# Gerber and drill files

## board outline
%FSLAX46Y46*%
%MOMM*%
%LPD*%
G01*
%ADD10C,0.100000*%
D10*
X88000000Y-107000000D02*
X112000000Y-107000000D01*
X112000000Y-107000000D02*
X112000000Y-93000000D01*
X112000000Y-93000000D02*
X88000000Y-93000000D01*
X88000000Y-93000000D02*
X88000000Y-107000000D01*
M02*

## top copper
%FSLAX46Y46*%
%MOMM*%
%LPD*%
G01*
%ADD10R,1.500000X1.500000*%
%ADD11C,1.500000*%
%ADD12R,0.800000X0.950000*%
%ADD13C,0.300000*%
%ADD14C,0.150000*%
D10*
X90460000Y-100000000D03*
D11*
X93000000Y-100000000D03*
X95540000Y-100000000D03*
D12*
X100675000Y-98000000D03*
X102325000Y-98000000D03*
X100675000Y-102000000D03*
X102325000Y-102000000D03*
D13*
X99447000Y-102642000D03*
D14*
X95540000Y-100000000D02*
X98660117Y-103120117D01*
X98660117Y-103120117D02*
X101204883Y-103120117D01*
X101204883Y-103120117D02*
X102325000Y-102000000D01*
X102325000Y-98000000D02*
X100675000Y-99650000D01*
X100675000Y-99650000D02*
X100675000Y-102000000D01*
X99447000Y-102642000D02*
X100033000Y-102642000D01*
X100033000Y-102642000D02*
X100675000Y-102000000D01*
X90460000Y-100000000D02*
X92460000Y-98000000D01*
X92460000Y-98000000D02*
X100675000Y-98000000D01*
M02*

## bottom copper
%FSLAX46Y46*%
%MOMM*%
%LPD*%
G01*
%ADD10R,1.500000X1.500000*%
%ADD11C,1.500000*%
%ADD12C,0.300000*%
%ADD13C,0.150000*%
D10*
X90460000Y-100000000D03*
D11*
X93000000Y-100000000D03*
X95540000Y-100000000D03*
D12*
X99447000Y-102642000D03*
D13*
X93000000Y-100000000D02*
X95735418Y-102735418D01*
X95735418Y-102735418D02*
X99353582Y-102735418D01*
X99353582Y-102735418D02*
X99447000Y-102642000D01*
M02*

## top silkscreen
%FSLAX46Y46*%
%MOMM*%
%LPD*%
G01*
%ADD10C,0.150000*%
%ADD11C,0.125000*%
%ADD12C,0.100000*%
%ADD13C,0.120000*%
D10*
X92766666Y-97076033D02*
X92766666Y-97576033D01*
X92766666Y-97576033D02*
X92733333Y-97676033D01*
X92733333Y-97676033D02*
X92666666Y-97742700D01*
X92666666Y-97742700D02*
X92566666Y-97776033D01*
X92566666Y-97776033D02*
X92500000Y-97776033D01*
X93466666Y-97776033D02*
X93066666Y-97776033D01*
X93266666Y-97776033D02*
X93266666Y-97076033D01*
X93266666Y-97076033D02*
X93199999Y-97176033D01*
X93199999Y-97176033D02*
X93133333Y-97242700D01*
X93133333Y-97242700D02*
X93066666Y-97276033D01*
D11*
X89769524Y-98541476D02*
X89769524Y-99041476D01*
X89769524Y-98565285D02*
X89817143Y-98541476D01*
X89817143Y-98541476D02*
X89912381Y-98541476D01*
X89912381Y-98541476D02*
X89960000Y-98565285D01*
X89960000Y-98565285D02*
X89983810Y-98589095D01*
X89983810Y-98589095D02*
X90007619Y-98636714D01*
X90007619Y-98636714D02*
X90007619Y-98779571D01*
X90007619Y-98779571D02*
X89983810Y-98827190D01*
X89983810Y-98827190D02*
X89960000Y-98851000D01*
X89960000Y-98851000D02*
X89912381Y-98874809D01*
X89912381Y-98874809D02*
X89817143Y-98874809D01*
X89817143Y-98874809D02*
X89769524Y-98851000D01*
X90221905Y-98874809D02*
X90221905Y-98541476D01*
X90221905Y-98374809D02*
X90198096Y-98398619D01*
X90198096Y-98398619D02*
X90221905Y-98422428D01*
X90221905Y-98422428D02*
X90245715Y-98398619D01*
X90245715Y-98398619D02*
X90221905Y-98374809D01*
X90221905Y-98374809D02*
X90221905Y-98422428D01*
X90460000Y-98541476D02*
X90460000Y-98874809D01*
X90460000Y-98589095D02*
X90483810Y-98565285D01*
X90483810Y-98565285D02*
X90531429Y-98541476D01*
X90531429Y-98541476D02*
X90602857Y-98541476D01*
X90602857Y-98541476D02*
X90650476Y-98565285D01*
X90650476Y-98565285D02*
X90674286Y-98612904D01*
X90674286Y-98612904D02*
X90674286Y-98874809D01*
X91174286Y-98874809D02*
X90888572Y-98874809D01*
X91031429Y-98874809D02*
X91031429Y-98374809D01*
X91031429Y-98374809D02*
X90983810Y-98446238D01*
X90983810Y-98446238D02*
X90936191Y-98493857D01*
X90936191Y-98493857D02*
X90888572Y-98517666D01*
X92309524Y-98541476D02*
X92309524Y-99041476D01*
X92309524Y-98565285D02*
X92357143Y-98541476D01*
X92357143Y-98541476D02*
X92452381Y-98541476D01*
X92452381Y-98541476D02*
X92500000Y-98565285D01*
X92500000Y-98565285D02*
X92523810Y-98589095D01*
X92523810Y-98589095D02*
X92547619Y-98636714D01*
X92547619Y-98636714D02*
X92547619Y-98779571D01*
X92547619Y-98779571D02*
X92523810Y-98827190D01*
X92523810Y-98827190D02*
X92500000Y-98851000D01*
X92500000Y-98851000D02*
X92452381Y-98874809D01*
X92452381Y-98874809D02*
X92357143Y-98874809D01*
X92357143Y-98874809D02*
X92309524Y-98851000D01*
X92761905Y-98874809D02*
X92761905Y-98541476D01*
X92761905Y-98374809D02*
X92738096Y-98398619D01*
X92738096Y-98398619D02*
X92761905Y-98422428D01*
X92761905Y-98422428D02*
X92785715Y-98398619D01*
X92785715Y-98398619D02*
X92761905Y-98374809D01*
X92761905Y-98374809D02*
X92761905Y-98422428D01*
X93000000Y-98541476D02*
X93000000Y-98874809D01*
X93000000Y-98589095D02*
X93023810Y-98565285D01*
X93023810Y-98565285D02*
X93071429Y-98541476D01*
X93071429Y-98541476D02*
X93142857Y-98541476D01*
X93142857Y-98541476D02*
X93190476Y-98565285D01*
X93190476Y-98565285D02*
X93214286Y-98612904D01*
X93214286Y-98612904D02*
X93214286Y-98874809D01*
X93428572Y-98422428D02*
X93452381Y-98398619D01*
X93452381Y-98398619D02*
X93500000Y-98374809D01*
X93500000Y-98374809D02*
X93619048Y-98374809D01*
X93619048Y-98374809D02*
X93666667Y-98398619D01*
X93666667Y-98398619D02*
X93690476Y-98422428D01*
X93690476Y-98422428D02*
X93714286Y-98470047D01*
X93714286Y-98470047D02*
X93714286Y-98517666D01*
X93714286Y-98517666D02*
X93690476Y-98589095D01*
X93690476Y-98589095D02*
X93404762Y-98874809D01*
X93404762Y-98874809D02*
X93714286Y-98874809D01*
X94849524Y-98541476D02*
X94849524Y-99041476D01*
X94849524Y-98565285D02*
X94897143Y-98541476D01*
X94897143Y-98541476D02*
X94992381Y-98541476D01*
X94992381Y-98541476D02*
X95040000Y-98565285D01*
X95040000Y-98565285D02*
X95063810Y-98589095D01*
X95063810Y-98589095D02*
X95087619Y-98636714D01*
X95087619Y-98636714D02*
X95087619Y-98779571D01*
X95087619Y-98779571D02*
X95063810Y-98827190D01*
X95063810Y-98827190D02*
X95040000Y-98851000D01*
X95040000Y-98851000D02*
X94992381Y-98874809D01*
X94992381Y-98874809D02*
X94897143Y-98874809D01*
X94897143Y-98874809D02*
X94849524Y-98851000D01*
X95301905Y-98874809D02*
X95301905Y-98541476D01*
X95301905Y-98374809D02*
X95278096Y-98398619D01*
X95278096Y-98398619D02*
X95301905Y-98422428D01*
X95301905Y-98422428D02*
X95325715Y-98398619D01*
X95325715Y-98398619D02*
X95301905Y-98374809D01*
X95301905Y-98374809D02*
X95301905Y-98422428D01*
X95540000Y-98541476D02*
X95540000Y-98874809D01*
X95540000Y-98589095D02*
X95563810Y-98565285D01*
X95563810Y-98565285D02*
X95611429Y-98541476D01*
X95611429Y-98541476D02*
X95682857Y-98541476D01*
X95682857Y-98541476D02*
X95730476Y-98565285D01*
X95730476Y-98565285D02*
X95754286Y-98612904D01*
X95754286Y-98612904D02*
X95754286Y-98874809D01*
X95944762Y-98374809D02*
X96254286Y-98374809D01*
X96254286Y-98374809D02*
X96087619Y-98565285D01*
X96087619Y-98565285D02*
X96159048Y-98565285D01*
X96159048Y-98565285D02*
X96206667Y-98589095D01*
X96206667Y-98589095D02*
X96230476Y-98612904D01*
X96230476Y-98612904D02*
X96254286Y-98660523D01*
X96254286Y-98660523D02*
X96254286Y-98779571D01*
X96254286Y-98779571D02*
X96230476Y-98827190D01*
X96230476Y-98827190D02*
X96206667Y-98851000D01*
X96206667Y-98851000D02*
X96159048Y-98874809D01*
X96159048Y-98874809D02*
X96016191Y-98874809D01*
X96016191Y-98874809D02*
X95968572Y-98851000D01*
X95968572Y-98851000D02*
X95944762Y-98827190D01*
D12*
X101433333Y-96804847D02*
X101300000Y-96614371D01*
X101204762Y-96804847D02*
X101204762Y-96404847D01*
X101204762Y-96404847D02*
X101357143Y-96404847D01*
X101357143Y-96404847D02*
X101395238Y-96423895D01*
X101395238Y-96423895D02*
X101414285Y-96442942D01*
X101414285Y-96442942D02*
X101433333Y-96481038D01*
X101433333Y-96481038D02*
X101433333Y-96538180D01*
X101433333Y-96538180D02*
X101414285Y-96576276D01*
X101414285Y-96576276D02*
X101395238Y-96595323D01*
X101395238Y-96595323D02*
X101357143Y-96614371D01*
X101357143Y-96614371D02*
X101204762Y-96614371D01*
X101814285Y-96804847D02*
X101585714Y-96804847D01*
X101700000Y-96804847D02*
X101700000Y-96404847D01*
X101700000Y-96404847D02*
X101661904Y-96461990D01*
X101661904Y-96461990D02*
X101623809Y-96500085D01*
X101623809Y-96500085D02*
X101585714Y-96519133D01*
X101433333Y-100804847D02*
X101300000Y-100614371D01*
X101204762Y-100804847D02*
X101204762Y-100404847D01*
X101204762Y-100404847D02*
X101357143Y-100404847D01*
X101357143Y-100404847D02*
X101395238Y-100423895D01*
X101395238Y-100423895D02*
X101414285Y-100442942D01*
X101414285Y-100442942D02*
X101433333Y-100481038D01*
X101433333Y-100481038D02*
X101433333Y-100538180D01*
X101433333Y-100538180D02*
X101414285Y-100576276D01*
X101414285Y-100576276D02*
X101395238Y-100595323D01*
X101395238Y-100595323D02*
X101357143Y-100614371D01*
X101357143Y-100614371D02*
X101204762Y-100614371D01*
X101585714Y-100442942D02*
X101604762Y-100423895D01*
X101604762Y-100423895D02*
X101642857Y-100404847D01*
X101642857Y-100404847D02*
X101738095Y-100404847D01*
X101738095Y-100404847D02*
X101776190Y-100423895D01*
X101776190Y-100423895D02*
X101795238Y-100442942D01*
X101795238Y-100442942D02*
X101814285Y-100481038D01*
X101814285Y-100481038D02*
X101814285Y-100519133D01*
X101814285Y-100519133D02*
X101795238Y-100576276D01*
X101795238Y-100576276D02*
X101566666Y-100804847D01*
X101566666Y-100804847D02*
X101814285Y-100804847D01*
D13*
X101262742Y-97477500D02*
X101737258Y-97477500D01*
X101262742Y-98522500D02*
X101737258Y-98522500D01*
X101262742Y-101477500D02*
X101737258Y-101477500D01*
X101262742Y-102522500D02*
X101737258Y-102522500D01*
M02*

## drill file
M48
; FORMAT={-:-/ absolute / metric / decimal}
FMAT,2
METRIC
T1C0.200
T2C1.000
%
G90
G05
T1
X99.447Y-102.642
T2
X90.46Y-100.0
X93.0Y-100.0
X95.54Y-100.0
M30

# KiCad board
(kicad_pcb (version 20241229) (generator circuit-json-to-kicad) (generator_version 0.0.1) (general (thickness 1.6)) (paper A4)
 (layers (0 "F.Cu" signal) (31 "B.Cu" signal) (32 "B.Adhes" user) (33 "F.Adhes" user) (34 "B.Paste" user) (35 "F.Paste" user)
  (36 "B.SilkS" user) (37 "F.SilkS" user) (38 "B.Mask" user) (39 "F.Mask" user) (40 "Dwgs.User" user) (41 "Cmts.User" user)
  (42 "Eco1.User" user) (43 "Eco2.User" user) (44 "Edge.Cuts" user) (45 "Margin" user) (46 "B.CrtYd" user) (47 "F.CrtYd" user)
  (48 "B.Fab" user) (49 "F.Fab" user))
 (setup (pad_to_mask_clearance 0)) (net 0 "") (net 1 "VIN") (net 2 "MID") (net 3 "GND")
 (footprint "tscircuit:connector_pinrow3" (layer F.Cu) (at 93 100 0)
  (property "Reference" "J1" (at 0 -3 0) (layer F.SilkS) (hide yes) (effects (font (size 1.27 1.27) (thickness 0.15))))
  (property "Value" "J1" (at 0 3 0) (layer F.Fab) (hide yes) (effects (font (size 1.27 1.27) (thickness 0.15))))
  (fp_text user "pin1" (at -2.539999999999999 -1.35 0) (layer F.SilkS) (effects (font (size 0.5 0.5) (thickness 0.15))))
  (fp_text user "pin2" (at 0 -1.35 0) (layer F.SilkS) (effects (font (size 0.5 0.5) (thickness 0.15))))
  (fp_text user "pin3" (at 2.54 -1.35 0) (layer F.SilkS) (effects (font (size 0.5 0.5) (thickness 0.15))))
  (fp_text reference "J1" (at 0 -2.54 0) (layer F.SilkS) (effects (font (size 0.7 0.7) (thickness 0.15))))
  (pad "1" thru_hole rect (at -2.539999999999999 0 0) (size 1.5 1.5) (drill 1) (layers *.Cu *.Mask) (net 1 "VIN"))
  (pad "2" thru_hole circle (at 0 0 0) (size 1.5 1.5) (drill 1) (layers *.Cu *.Mask) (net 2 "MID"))
  (pad "3" thru_hole circle (at 2.54 0 0) (size 1.5 1.5) (drill 1) (layers *.Cu *.Mask) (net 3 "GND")))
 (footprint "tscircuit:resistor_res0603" (layer F.Cu) (at 101.5 98 0)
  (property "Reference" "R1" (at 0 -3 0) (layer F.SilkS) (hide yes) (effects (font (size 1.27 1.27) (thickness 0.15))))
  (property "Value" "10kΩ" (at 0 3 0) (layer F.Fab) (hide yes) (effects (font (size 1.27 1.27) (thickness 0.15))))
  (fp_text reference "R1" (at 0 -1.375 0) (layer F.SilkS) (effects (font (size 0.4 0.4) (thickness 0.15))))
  (fp_line (start -0.23725799999999997 -0.5225) (end 0.23725799999999997 -0.5225) (stroke (width 0.12) (type default)) (layer F.SilkS))
  (fp_line (start -0.23725799999999997 0.5225) (end 0.23725799999999997 0.5225) (stroke (width 0.12) (type default)) (layer F.SilkS))
  (pad "1" smd rect (at -0.825 0 0) (size 0.8 0.95) (layers F.Cu F.Mask) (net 1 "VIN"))
  (pad "2" smd rect (at 0.8250000000000002 0 0) (size 0.8 0.95) (layers F.Cu F.Mask) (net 2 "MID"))
  (pad "" smd rect (at -0.825 0 0) (size 0.5599999999999999 0.6649999999999999) (layers F.Paste))
  (pad "" smd rect (at 0.8250000000000002 0 0) (size 0.5599999999999999 0.6649999999999999) (layers F.Paste)))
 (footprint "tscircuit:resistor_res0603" (layer F.Cu) (at 101.5 102 0)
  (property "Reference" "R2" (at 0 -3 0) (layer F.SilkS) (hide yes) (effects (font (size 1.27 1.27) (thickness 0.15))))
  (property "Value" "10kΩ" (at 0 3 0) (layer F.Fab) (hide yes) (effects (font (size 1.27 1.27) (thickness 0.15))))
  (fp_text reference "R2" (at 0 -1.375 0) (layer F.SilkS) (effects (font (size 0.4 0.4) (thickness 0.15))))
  (fp_line (start -0.23725799999999997 -0.5225) (end 0.23725799999999997 -0.5225) (stroke (width 0.12) (type default)) (layer F.SilkS))
  (fp_line (start -0.23725799999999997 0.5225) (end 0.23725799999999997 0.5225) (stroke (width 0.12) (type default)) (layer F.SilkS))
  (pad "1" smd rect (at -0.825 0 0) (size 0.8 0.95) (layers F.Cu F.Mask) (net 2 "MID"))
  (pad "2" smd rect (at 0.8250000000000002 0 0) (size 0.8 0.95) (layers F.Cu F.Mask) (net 3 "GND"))
  (pad "" smd rect (at -0.825 0 0) (size 0.5599999999999999 0.6649999999999999) (layers F.Paste))
  (pad "" smd rect (at 0.8250000000000002 0 0) (size 0.5599999999999999 0.6649999999999999) (layers F.Paste)))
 (segment (start 95.54 100) (end 98.66011723078628 103.12011723078629) (width 0.15) (layer F.Cu) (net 3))
 (segment (start 98.66011723078628 103.12011723078629) (end 101.20488276921371 103.12011723078629) (width 0.15) (layer F.Cu) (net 3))
 (segment (start 101.20488276921371 103.12011723078629) (end 102.325 102) (width 0.15) (layer F.Cu) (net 3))
 (segment (start 102.325 98) (end 100.675 99.65) (width 0.15) (layer F.Cu) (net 2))
 (segment (start 100.675 99.65) (end 100.675 102) (width 0.15) (layer F.Cu) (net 2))
 (segment (start 93 100) (end 95.73541811585916 102.73541811585916) (width 0.15) (layer B.Cu) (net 2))
 (segment (start 95.73541811585916 102.73541811585916) (end 99.35358188414084 102.73541811585916) (width 0.15) (layer B.Cu) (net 2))
 (segment (start 99.35358188414084 102.73541811585916) (end 99.447 102.642) (width 0.15) (layer B.Cu) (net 2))
 (segment (start 99.447 102.642) (end 100.033 102.642) (width 0.15) (layer F.Cu) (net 2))
 (segment (start 100.033 102.642) (end 100.675 102) (width 0.15) (layer F.Cu) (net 2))
 (segment (start 90.46000000000001 100) (end 92.46000000000001 98) (width 0.15) (layer F.Cu) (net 1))
 (segment (start 92.46000000000001 98) (end 100.675 98) (width 0.15) (layer F.Cu) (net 1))
 (gr_line (start 88 107) (end 112 107) (width 0.1) (layer Edge.Cuts))
 (gr_line (start 112 107) (end 112 93) (width 0.1) (layer Edge.Cuts))
 (gr_line (start 112 93) (end 88 93) (width 0.1) (layer Edge.Cuts))
 (gr_line (start 88 93) (end 88 107) (width 0.1) (layer Edge.Cuts))
 (via (at 99.447 102.642) (size 0.3) (drill 0.2) (layers F.Cu B.Cu) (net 2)))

